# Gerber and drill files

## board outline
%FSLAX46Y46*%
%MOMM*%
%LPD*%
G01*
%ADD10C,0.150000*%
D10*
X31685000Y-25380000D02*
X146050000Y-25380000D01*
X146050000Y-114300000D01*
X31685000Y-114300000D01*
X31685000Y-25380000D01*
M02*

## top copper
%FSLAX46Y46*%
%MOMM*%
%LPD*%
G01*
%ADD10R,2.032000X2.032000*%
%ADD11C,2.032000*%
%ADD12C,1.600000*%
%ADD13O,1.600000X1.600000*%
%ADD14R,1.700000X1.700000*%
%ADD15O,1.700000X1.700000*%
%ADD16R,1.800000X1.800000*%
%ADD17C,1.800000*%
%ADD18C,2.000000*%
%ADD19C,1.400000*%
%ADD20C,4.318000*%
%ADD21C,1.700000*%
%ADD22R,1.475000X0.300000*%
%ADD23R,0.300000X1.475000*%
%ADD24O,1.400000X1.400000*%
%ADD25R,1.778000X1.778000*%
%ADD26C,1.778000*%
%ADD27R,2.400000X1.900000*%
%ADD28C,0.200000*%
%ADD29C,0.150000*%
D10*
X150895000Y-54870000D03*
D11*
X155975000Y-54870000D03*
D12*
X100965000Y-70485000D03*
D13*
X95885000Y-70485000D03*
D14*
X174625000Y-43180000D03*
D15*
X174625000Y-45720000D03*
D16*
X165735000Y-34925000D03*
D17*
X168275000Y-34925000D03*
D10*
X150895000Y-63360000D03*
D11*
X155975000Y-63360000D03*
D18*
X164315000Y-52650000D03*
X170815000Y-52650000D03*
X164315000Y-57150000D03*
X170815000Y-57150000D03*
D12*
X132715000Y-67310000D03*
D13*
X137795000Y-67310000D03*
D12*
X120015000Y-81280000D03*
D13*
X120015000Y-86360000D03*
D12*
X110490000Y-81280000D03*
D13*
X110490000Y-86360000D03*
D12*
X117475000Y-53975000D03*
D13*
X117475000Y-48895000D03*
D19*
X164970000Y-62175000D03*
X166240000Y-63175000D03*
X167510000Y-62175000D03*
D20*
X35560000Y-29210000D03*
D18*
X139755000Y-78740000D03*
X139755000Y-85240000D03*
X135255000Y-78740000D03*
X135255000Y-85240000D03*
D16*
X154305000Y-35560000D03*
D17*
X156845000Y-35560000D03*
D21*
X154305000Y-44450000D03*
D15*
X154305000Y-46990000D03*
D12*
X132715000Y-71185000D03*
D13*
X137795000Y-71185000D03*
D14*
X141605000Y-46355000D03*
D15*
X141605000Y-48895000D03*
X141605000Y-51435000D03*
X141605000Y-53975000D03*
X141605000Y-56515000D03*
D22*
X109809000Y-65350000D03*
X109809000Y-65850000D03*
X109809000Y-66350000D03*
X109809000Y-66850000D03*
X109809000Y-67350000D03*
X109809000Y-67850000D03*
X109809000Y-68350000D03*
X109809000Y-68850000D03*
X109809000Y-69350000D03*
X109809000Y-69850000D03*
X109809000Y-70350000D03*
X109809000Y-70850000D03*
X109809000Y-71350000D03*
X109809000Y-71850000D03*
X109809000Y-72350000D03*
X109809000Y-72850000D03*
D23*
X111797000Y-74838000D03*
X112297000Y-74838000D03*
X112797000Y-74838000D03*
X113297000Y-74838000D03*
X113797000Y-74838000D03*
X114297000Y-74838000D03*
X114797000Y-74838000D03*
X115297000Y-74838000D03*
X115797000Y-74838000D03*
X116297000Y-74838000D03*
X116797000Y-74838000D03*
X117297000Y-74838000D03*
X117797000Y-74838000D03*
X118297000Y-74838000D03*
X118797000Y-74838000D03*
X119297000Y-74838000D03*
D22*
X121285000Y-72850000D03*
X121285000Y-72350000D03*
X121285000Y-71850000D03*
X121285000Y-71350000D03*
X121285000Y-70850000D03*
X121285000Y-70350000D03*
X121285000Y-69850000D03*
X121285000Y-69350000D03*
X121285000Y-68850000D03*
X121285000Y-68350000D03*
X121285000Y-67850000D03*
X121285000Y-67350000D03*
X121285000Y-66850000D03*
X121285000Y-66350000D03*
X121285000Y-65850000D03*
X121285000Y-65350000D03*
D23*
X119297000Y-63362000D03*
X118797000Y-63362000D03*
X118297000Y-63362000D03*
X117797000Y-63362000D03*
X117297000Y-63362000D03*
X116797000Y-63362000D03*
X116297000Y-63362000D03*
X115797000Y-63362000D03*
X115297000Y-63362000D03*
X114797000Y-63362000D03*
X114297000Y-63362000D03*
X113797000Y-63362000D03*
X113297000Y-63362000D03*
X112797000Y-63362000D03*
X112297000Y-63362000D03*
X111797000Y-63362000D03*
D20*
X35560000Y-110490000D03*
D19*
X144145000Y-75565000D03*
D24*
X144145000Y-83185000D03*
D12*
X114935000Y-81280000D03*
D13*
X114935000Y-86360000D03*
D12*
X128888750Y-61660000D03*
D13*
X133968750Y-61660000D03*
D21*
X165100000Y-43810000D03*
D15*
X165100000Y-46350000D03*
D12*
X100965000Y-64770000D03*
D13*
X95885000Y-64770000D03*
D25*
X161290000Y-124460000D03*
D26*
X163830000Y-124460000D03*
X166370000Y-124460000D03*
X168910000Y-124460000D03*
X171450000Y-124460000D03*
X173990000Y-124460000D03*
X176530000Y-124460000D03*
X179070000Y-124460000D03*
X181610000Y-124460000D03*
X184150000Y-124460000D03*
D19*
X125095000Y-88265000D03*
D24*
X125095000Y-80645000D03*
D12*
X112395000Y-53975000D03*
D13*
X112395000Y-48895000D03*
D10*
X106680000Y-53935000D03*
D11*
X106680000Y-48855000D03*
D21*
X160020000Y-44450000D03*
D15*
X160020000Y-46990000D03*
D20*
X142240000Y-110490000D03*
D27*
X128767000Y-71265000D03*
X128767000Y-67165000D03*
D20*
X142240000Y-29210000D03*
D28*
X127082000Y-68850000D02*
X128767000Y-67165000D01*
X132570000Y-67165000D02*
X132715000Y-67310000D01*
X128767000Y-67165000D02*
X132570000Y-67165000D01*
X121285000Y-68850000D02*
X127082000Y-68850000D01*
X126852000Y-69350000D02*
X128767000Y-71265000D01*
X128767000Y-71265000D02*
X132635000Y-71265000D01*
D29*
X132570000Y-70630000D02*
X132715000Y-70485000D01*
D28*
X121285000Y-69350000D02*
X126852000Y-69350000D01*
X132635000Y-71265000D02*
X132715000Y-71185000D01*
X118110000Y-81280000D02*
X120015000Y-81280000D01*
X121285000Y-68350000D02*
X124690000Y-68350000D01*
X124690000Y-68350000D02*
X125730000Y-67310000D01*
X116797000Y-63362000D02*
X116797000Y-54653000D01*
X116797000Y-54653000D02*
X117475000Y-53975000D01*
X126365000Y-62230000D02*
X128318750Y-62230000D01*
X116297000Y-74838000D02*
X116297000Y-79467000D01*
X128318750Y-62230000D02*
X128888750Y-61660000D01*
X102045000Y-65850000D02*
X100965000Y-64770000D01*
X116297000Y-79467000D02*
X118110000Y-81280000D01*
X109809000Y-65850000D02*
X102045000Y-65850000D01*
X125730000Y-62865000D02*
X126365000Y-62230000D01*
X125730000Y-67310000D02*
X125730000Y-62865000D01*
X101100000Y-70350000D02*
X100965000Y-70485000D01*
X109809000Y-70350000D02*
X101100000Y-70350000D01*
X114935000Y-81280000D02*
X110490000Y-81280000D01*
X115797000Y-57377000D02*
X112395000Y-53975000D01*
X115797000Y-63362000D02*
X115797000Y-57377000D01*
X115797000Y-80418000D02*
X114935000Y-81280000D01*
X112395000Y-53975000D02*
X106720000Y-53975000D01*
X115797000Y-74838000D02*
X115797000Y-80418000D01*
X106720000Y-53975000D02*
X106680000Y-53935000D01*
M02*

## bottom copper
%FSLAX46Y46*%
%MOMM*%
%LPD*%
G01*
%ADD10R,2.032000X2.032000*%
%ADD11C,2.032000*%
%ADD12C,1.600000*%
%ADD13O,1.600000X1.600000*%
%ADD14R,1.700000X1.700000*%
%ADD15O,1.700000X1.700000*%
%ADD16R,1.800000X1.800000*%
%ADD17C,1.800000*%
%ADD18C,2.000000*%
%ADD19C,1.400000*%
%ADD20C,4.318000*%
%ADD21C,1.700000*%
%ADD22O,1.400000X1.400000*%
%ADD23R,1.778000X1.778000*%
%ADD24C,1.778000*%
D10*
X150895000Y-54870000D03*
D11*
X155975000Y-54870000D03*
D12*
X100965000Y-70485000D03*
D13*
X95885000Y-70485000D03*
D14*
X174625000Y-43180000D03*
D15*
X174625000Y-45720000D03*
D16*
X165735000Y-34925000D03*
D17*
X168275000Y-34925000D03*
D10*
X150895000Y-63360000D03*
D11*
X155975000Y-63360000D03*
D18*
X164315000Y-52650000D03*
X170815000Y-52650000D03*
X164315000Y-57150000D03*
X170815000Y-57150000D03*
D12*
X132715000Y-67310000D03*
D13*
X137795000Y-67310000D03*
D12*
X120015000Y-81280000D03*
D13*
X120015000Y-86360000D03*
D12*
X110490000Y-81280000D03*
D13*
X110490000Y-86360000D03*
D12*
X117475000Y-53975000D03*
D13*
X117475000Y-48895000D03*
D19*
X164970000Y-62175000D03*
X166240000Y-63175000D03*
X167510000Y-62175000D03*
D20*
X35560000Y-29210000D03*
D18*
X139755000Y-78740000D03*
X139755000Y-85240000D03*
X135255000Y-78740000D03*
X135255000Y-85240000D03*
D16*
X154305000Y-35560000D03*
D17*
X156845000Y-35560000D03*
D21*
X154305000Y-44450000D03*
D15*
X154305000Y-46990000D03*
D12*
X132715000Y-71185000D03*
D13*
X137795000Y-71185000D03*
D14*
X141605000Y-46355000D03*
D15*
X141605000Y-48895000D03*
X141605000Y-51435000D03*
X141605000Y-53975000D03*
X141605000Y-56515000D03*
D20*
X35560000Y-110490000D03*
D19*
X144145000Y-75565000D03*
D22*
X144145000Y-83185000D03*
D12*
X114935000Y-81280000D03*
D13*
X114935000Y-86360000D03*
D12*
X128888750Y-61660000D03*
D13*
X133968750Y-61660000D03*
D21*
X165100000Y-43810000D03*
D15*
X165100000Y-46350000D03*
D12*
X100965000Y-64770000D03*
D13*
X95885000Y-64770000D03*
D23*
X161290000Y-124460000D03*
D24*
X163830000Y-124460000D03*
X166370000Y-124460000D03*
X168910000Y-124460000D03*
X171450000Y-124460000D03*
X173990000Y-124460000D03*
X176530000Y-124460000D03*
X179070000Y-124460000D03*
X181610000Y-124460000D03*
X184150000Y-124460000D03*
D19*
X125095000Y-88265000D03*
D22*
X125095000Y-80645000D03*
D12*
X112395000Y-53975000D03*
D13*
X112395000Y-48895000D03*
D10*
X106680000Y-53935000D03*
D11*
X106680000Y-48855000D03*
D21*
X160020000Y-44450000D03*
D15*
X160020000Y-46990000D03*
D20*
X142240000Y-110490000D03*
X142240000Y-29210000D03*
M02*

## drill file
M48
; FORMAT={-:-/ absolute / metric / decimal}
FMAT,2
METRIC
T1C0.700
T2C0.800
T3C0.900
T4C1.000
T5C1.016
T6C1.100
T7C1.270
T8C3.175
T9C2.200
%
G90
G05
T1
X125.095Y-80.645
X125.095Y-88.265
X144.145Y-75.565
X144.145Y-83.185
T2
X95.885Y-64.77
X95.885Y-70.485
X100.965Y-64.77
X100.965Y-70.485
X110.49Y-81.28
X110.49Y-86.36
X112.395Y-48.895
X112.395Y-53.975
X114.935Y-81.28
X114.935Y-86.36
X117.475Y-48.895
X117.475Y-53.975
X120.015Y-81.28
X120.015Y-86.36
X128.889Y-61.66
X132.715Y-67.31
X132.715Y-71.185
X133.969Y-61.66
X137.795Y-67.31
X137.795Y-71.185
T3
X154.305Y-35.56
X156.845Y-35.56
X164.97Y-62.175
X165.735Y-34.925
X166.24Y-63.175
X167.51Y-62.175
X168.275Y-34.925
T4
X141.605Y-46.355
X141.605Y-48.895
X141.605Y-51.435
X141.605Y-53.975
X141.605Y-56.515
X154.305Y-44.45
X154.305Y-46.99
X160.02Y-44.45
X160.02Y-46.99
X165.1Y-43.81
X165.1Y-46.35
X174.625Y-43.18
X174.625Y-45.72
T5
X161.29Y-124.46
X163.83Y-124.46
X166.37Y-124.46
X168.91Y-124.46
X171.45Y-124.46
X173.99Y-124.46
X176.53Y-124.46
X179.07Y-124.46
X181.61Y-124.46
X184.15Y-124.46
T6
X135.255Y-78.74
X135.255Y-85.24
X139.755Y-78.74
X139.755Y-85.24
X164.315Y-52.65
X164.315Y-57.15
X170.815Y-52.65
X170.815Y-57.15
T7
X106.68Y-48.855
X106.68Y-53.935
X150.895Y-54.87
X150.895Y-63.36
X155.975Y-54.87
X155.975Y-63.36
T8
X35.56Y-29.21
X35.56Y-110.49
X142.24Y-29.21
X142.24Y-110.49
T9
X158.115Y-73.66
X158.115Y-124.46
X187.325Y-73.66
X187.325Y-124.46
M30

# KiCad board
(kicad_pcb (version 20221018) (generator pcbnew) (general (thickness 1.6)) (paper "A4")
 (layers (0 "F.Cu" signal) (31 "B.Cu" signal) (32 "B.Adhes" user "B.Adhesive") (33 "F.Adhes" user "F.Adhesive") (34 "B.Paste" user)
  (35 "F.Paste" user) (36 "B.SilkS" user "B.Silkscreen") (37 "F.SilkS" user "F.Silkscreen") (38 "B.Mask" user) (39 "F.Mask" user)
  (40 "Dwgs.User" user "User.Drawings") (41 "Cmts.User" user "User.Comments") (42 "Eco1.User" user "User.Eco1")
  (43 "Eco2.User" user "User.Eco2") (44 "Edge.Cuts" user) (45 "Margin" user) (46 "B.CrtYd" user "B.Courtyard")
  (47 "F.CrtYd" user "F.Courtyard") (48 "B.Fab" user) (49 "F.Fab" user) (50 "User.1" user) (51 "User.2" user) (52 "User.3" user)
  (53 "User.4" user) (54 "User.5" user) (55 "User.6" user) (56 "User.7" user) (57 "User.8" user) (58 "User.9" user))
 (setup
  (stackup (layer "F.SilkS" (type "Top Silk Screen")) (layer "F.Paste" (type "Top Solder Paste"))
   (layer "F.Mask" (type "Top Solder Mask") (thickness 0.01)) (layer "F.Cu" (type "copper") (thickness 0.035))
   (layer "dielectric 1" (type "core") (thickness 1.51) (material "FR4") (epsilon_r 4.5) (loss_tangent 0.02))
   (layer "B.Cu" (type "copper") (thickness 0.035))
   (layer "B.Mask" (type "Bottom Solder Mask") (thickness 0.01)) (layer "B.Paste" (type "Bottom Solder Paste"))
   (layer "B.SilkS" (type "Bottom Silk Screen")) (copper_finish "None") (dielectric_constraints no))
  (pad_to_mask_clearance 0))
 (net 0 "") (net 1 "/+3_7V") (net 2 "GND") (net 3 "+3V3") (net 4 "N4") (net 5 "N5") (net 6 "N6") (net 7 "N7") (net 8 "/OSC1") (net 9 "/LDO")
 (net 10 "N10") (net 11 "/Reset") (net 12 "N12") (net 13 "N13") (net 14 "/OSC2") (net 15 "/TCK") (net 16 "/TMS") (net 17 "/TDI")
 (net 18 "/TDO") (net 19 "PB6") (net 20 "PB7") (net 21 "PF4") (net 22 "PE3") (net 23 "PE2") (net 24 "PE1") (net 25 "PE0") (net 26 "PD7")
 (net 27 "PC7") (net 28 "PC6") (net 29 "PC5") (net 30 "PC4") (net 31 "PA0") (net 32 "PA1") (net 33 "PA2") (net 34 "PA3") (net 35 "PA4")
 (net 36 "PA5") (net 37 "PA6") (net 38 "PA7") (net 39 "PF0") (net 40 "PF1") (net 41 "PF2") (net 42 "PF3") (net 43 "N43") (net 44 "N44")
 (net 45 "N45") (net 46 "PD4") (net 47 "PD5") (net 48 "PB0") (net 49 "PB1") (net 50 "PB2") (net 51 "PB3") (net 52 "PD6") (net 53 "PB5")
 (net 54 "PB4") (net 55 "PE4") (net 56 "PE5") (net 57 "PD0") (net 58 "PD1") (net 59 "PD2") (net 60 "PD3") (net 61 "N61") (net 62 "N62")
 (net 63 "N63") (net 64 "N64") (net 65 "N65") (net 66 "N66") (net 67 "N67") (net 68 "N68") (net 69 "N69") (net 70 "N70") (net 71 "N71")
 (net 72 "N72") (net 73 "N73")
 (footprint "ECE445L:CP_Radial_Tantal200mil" (layer "F.Cu") (at 150.895 54.87)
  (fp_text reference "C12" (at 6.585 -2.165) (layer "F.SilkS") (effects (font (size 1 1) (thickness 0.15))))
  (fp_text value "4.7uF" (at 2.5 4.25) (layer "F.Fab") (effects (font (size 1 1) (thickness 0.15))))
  (pad "1" thru_hole rect (at 0 0) (size 2.032 2.032) (drill 1.27) (layers "*.Cu" "*.Mask") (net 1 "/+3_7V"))
  (pad "2" thru_hole circle (at 5.08 0) (size 2.032 2.032) (drill 1.27) (layers "*.Cu" "*.Mask") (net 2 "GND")))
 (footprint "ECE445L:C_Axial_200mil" (layer "F.Cu") (at 100.965 70.485 180)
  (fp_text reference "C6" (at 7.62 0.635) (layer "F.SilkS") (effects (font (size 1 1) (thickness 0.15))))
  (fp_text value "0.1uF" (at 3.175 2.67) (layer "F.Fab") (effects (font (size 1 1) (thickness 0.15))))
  (pad "1" thru_hole circle (at 0 0 180) (size 1.6 1.6) (drill 0.8) (layers "*.Cu" "*.Mask") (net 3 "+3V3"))
  (pad "2" thru_hole oval (at 5.08 0 180) (size 1.6 1.6) (drill 0.8) (layers "*.Cu" "*.Mask") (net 2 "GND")))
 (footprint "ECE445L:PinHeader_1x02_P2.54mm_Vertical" (layer "F.Cu") (at 174.625 43.18)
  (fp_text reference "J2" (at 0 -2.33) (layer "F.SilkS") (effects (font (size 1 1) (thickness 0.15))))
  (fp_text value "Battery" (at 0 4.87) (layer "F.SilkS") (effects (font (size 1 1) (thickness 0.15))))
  (pad "1" thru_hole rect (at 0 0) (size 1.7 1.7) (drill 1) (layers "*.Cu" "*.Mask") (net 2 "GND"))
  (pad "2" thru_hole oval (at 0 2.54) (size 1.7 1.7) (drill 1) (layers "*.Cu" "*.Mask") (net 1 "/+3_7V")))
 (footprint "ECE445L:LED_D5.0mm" (layer "F.Cu") (at 165.735 34.925)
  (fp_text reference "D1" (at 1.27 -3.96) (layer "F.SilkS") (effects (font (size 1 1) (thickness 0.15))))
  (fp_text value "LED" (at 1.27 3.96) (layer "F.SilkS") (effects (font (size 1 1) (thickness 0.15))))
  (pad "1" thru_hole rect (at 0 0) (size 1.8 1.8) (drill 0.9) (layers "*.Cu" "*.Mask") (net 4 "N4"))
  (pad "2" thru_hole circle (at 2.54 0) (size 1.8 1.8) (drill 0.9) (layers "*.Cu" "*.Mask") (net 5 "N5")))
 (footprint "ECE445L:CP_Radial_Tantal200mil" (layer "F.Cu") (at 150.895 63.36)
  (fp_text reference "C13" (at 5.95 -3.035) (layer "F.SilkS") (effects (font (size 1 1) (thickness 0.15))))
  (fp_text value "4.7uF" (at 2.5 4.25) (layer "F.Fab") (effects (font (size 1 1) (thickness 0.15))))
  (pad "1" thru_hole rect (at 0 0) (size 2.032 2.032) (drill 1.27) (layers "*.Cu" "*.Mask") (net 3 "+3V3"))
  (pad "2" thru_hole circle (at 5.08 0) (size 2.032 2.032) (drill 1.27) (layers "*.Cu" "*.Mask") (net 2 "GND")))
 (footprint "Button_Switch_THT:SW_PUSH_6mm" (layer "F.Cu") (at 164.315 52.65)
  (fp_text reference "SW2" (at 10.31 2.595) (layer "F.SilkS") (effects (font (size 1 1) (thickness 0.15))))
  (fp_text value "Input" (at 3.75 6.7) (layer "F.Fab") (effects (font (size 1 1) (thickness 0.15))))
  (pad "1" thru_hole circle (at 0 0 90) (size 2 2) (drill 1.1) (layers "*.Cu" "*.Mask") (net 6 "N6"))
  (pad "1" thru_hole circle (at 6.5 0 90) (size 2 2) (drill 1.1) (layers "*.Cu" "*.Mask") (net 6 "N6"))
  (pad "2" thru_hole circle (at 0 4.5 90) (size 2 2) (drill 1.1) (layers "*.Cu" "*.Mask") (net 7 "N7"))
  (pad "2" thru_hole circle (at 6.5 4.5 90) (size 2 2) (drill 1.1) (layers "*.Cu" "*.Mask") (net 7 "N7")))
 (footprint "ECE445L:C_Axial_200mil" (layer "F.Cu") (at 132.715 67.31)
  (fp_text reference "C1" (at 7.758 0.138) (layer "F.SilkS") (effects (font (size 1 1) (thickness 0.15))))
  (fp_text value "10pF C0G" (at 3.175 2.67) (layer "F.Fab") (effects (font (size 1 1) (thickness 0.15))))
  (pad "1" thru_hole circle (at 0 0) (size 1.6 1.6) (drill 0.8) (layers "*.Cu" "*.Mask") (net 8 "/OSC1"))
  (pad "2" thru_hole oval (at 5.08 0) (size 1.6 1.6) (drill 0.8) (layers "*.Cu" "*.Mask") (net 2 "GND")))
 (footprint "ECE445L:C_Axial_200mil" (layer "F.Cu") (at 120.015 81.28 -90)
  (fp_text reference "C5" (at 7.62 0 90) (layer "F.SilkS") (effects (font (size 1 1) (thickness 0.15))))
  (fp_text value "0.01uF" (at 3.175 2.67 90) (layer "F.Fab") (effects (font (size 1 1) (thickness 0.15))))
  (pad "1" thru_hole circle (at 0 0 270) (size 1.6 1.6) (drill 0.8) (layers "*.Cu" "*.Mask") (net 3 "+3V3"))
  (pad "2" thru_hole oval (at 5.08 0 270) (size 1.6 1.6) (drill 0.8) (layers "*.Cu" "*.Mask") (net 2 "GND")))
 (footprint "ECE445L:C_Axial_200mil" (layer "F.Cu") (at 110.49 81.28 -90)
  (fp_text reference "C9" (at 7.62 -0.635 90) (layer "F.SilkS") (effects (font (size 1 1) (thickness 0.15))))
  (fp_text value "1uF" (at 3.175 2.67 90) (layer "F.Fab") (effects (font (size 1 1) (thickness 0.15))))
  (pad "1" thru_hole circle (at 0 0 270) (size 1.6 1.6) (drill 0.8) (layers "*.Cu" "*.Mask") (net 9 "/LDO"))
  (pad "2" thru_hole oval (at 5.08 0 270) (size 1.6 1.6) (drill 0.8) (layers "*.Cu" "*.Mask") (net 2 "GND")))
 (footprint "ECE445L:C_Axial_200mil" (layer "F.Cu") (at 117.475 53.975 90)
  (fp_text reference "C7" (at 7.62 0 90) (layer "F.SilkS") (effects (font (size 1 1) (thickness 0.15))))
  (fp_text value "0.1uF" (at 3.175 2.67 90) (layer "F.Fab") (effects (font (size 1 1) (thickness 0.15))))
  (pad "1" thru_hole circle (at 0 0 90) (size 1.6 1.6) (drill 0.8) (layers "*.Cu" "*.Mask") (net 3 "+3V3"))
  (pad "2" thru_hole oval (at 5.08 0 90) (size 1.6 1.6) (drill 0.8) (layers "*.Cu" "*.Mask") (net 2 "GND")))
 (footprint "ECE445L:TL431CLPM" (layer "F.Cu") (at 164.97 62.175)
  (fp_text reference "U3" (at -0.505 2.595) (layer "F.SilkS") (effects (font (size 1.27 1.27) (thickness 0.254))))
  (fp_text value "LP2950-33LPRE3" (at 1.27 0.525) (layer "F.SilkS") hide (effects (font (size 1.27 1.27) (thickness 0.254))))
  (pad "1" thru_hole circle (at 0 0) (size 1.4 1.4) (drill 0.9) (layers "*.Cu" "*.Mask") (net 3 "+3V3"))
  (pad "2" thru_hole circle (at 1.27 1) (size 1.4 1.4) (drill 0.9) (layers "*.Cu" "*.Mask") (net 2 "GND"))
  (pad "3" thru_hole circle (at 2.54 0) (size 1.4 1.4) (drill 0.9) (layers "*.Cu" "*.Mask") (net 1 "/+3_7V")))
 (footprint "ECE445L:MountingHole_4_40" (layer "F.Cu") (at 35.56 29.21)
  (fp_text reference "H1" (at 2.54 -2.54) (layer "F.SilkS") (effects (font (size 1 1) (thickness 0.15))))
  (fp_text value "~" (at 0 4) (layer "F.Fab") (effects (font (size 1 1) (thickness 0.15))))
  (pad "1" thru_hole circle (at 0 0) (size 4.318 4.318) (drill 3.175) (layers "*.Cu" "*.Mask") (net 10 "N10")))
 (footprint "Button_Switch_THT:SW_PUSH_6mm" (layer "F.Cu") (at 139.755 78.74 -90)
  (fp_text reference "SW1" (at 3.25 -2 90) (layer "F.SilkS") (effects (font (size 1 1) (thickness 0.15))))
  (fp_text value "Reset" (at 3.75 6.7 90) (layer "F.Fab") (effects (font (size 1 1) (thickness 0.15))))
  (pad "1" thru_hole circle (at 0 0) (size 2 2) (drill 1.1) (layers "*.Cu" "*.Mask") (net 2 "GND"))
  (pad "1" thru_hole circle (at 6.5 0) (size 2 2) (drill 1.1) (layers "*.Cu" "*.Mask") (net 2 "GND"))
  (pad "2" thru_hole circle (at 0 4.5) (size 2 2) (drill 1.1) (layers "*.Cu" "*.Mask") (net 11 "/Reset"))
  (pad "2" thru_hole circle (at 6.5 4.5) (size 2 2) (drill 1.1) (layers "*.Cu" "*.Mask") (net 11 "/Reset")))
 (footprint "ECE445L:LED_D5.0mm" (layer "F.Cu") (at 154.305 35.56)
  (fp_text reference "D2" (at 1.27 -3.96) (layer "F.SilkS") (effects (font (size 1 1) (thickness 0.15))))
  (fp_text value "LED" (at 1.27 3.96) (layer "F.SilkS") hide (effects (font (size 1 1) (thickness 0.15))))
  (pad "1" thru_hole rect (at 0 0) (size 1.8 1.8) (drill 0.9) (layers "*.Cu" "*.Mask") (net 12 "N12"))
  (pad "2" thru_hole circle (at 2.54 0) (size 1.8 1.8) (drill 0.9) (layers "*.Cu" "*.Mask") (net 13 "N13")))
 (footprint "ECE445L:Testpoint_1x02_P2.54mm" (layer "F.Cu") (at 154.305 44.45)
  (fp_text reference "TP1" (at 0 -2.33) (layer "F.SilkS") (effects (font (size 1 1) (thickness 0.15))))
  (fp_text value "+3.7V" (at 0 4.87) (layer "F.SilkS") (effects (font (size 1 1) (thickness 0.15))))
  (pad "1" thru_hole circle (at 0 0) (size 1.7 1.7) (drill 1) (layers "*.Cu" "*.Mask") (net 1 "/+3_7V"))
  (pad "2" thru_hole oval (at 0 2.54) (size 1.7 1.7) (drill 1) (layers "*.Cu" "*.Mask") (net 1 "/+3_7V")))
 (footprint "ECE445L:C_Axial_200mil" (layer "F.Cu") (at 132.715 71.185)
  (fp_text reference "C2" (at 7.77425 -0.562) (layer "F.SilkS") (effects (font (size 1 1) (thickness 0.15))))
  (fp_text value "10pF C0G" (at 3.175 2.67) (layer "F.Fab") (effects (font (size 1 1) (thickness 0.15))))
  (pad "1" thru_hole circle (at 0 0) (size 1.6 1.6) (drill 0.8) (layers "*.Cu" "*.Mask") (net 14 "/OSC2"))
  (pad "2" thru_hole oval (at 5.08 0) (size 1.6 1.6) (drill 0.8) (layers "*.Cu" "*.Mask") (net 2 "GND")))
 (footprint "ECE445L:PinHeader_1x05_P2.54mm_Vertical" (layer "F.Cu") (at 141.605 46.355)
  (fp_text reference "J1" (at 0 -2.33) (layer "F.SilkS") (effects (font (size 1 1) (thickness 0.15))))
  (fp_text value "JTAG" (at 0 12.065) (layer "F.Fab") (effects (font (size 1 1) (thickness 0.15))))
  (pad "1" thru_hole rect (at 0 0) (size 1.7 1.7) (drill 1) (layers "*.Cu" "*.Mask") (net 2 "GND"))
  (pad "2" thru_hole oval (at 0 2.54) (size 1.7 1.7) (drill 1) (layers "*.Cu" "*.Mask") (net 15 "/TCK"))
  (pad "3" thru_hole oval (at 0 5.08) (size 1.7 1.7) (drill 1) (layers "*.Cu" "*.Mask") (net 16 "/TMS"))
  (pad "4" thru_hole oval (at 0 7.62) (size 1.7 1.7) (drill 1) (layers "*.Cu" "*.Mask") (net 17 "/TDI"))
  (pad "5" thru_hole oval (at 0 10.16) (size 1.7 1.7) (drill 1) (layers "*.Cu" "*.Mask") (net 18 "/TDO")))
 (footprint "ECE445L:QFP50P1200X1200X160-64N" (layer "F.Cu") (at 115.547 69.1)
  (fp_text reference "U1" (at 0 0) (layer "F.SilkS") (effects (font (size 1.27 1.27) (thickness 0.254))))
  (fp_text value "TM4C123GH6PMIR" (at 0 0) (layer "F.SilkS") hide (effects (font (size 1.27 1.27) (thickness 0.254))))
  (pad "1" smd rect (at -5.738 -3.75 90) (size 0.3 1.475) (layers "F.Cu" "F.Paste" "F.Mask") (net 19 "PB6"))
  (pad "2" smd rect (at -5.738 -3.25 90) (size 0.3 1.475) (layers "F.Cu" "F.Paste" "F.Mask") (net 3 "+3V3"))
  (pad "3" smd rect (at -5.738 -2.75 90) (size 0.3 1.475) (layers "F.Cu" "F.Paste" "F.Mask") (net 2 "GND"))
  (pad "4" smd rect (at -5.738 -2.25 90) (size 0.3 1.475) (layers "F.Cu" "F.Paste" "F.Mask") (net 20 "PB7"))
  (pad "5" smd rect (at -5.738 -1.75 90) (size 0.3 1.475) (layers "F.Cu" "F.Paste" "F.Mask") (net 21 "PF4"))
  (pad "6" smd rect (at -5.738 -1.25 90) (size 0.3 1.475) (layers "F.Cu" "F.Paste" "F.Mask") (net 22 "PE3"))
  (pad "7" smd rect (at -5.738 -0.75 90) (size 0.3 1.475) (layers "F.Cu" "F.Paste" "F.Mask") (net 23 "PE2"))
  (pad "8" smd rect (at -5.738 -0.25 90) (size 0.3 1.475) (layers "F.Cu" "F.Paste" "F.Mask") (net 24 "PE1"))
  (pad "9" smd rect (at -5.738 0.25 90) (size 0.3 1.475) (layers "F.Cu" "F.Paste" "F.Mask") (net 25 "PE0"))
  (pad "10" smd rect (at -5.738 0.75 90) (size 0.3 1.475) (layers "F.Cu" "F.Paste" "F.Mask") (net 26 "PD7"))
  (pad "11" smd rect (at -5.738 1.25 90) (size 0.3 1.475) (layers "F.Cu" "F.Paste" "F.Mask") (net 3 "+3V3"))
  (pad "12" smd rect (at -5.738 1.75 90) (size 0.3 1.475) (layers "F.Cu" "F.Paste" "F.Mask") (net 2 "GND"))
  (pad "13" smd rect (at -5.738 2.25 90) (size 0.3 1.475) (layers "F.Cu" "F.Paste" "F.Mask") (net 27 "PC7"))
  (pad "14" smd rect (at -5.738 2.75 90) (size 0.3 1.475) (layers "F.Cu" "F.Paste" "F.Mask") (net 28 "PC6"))
  (pad "15" smd rect (at -5.738 3.25 90) (size 0.3 1.475) (layers "F.Cu" "F.Paste" "F.Mask") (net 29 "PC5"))
  (pad "16" smd rect (at -5.738 3.75 90) (size 0.3 1.475) (layers "F.Cu" "F.Paste" "F.Mask") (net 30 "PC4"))
  (pad "17" smd rect (at -3.75 5.738) (size 0.3 1.475) (layers "F.Cu" "F.Paste" "F.Mask") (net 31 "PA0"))
  (pad "18" smd rect (at -3.25 5.738) (size 0.3 1.475) (layers "F.Cu" "F.Paste" "F.Mask") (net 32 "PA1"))
  (pad "19" smd rect (at -2.75 5.738) (size 0.3 1.475) (layers "F.Cu" "F.Paste" "F.Mask") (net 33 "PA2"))
  (pad "20" smd rect (at -2.25 5.738) (size 0.3 1.475) (layers "F.Cu" "F.Paste" "F.Mask") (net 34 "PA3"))
  (pad "21" smd rect (at -1.75 5.738) (size 0.3 1.475) (layers "F.Cu" "F.Paste" "F.Mask") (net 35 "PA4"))
  (pad "22" smd rect (at -1.25 5.738) (size 0.3 1.475) (layers "F.Cu" "F.Paste" "F.Mask") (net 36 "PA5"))
  (pad "23" smd rect (at -0.75 5.738) (size 0.3 1.475) (layers "F.Cu" "F.Paste" "F.Mask") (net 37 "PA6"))
  (pad "24" smd rect (at -0.25 5.738) (size 0.3 1.475) (layers "F.Cu" "F.Paste" "F.Mask") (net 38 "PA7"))
  (pad "25" smd rect (at 0.25 5.738) (size 0.3 1.475) (layers "F.Cu" "F.Paste" "F.Mask") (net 9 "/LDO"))
  (pad "26" smd rect (at 0.75 5.738) (size 0.3 1.475) (layers "F.Cu" "F.Paste" "F.Mask") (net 3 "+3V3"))
  (pad "27" smd rect (at 1.25 5.738) (size 0.3 1.475) (layers "F.Cu" "F.Paste" "F.Mask") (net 2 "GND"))
  (pad "28" smd rect (at 1.75 5.738) (size 0.3 1.475) (layers "F.Cu" "F.Paste" "F.Mask") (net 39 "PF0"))
  (pad "29" smd rect (at 2.25 5.738) (size 0.3 1.475) (layers "F.Cu" "F.Paste" "F.Mask") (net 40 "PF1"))
  (pad "30" smd rect (at 2.75 5.738) (size 0.3 1.475) (layers "F.Cu" "F.Paste" "F.Mask") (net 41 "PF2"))
  (pad "31" smd rect (at 3.25 5.738) (size 0.3 1.475) (layers "F.Cu" "F.Paste" "F.Mask") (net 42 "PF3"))
  (pad "32" smd rect (at 3.75 5.738) (size 0.3 1.475) (layers "F.Cu" "F.Paste" "F.Mask") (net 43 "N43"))
  (pad "33" smd rect (at 5.738 3.75 90) (size 0.3 1.475) (layers "F.Cu" "F.Paste" "F.Mask") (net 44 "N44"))
  (pad "34" smd rect (at 5.738 3.25 90) (size 0.3 1.475) (layers "F.Cu" "F.Paste" "F.Mask") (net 2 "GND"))
  (pad "35" smd rect (at 5.738 2.75 90) (size 0.3 1.475) (layers "F.Cu" "F.Paste" "F.Mask") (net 2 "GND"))
  (pad "36" smd rect (at 5.738 2.25 90) (size 0.3 1.475) (layers "F.Cu" "F.Paste" "F.Mask") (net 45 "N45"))
  (pad "37" smd rect (at 5.738 1.75 90) (size 0.3 1.475) (layers "F.Cu" "F.Paste" "F.Mask") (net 3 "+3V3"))
  (pad "38" smd rect (at 5.738 1.25 90) (size 0.3 1.475) (layers "F.Cu" "F.Paste" "F.Mask") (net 11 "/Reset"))
  (pad "39" smd rect (at 5.738 0.75 90) (size 0.3 1.475) (layers "F.Cu" "F.Paste" "F.Mask") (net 2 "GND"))
  (pad "40" smd rect (at 5.738 0.25 90) (size 0.3 1.475) (layers "F.Cu" "F.Paste" "F.Mask") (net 14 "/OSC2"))
  (pad "41" smd rect (at 5.738 -0.25 90) (size 0.3 1.475) (layers "F.Cu" "F.Paste" "F.Mask") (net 8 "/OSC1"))
  (pad "42" smd rect (at 5.738 -0.75 90) (size 0.3 1.475) (layers "F.Cu" "F.Paste" "F.Mask") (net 3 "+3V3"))
  (pad "43" smd rect (at 5.738 -1.25 90) (size 0.3 1.475) (layers "F.Cu" "F.Paste" "F.Mask") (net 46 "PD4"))
  (pad "44" smd rect (at 5.738 -1.75 90) (size 0.3 1.475) (layers "F.Cu" "F.Paste" "F.Mask") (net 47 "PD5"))
  (pad "45" smd rect (at 5.738 -2.25 90) (size 0.3 1.475) (layers "F.Cu" "F.Paste" "F.Mask") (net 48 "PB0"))
  (pad "46" smd rect (at 5.738 -2.75 90) (size 0.3 1.475) (layers "F.Cu" "F.Paste" "F.Mask") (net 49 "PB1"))
  (pad "47" smd rect (at 5.738 -3.25 90) (size 0.3 1.475) (layers "F.Cu" "F.Paste" "F.Mask") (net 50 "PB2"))
  (pad "48" smd rect (at 5.738 -3.75 90) (size 0.3 1.475) (layers "F.Cu" "F.Paste" "F.Mask") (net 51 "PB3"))
  (pad "49" smd rect (at 3.75 -5.738) (size 0.3 1.475) (layers "F.Cu" "F.Paste" "F.Mask") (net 18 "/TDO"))
  (pad "50" smd rect (at 3.25 -5.738) (size 0.3 1.475) (layers "F.Cu" "F.Paste" "F.Mask") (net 17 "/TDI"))
  (pad "51" smd rect (at 2.75 -5.738) (size 0.3 1.475) (layers "F.Cu" "F.Paste" "F.Mask") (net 16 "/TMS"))
  (pad "52" smd rect (at 2.25 -5.738) (size 0.3 1.475) (layers "F.Cu" "F.Paste" "F.Mask") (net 15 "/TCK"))
  (pad "53" smd rect (at 1.75 -5.738) (size 0.3 1.475) (layers "F.Cu" "F.Paste" "F.Mask") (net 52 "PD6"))
  (pad "54" smd rect (at 1.25 -5.738) (size 0.3 1.475) (layers "F.Cu" "F.Paste" "F.Mask") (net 3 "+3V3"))
  (pad "55" smd rect (at 0.75 -5.738) (size 0.3 1.475) (layers "F.Cu" "F.Paste" "F.Mask") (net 2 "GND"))
  (pad "56" smd rect (at 0.25 -5.738) (size 0.3 1.475) (layers "F.Cu" "F.Paste" "F.Mask") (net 9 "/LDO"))
  (pad "57" smd rect (at -0.25 -5.738) (size 0.3 1.475) (layers "F.Cu" "F.Paste" "F.Mask") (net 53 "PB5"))
  (pad "58" smd rect (at -0.75 -5.738) (size 0.3 1.475) (layers "F.Cu" "F.Paste" "F.Mask") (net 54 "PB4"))
  (pad "59" smd rect (at -1.25 -5.738) (size 0.3 1.475) (layers "F.Cu" "F.Paste" "F.Mask") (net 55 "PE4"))
  (pad "60" smd rect (at -1.75 -5.738) (size 0.3 1.475) (layers "F.Cu" "F.Paste" "F.Mask") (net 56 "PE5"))
  (pad "61" smd rect (at -2.25 -5.738) (size 0.3 1.475) (layers "F.Cu" "F.Paste" "F.Mask") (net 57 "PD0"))
  (pad "62" smd rect (at -2.75 -5.738) (size 0.3 1.475) (layers "F.Cu" "F.Paste" "F.Mask") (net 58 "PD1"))
  (pad "63" smd rect (at -3.25 -5.738) (size 0.3 1.475) (layers "F.Cu" "F.Paste" "F.Mask") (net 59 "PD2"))
  (pad "64" smd rect (at -3.75 -5.738) (size 0.3 1.475) (layers "F.Cu" "F.Paste" "F.Mask") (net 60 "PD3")))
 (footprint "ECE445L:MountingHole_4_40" (layer "F.Cu") (at 35.56 110.49)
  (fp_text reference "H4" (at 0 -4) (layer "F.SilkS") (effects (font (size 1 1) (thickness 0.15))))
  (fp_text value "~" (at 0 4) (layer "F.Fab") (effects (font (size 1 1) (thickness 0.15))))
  (pad "1" thru_hole circle (at 0 0) (size 4.318 4.318) (drill 3.175) (layers "*.Cu" "*.Mask") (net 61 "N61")))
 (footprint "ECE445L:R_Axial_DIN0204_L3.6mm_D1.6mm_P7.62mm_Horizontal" (layer "F.Cu") (at 144.145 75.565 -90)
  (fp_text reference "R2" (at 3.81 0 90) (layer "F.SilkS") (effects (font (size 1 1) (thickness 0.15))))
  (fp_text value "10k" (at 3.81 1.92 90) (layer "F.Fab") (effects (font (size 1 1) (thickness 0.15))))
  (pad "1" thru_hole circle (at 0 0 270) (size 1.4 1.4) (drill 0.7) (layers "*.Cu" "*.Mask") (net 3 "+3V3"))
  (pad "2" thru_hole oval (at 7.62 0 270) (size 1.4 1.4) (drill 0.7) (layers "*.Cu" "*.Mask") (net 11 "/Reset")))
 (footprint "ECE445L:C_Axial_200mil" (layer "F.Cu") (at 114.935 81.28 -90)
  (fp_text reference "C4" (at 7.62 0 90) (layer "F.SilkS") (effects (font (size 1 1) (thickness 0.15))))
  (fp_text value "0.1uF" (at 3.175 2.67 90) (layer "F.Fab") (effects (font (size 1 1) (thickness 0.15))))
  (pad "1" thru_hole circle (at 0 0 270) (size 1.6 1.6) (drill 0.8) (layers "*.Cu" "*.Mask") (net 9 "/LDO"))
  (pad "2" thru_hole oval (at 5.08 0 270) (size 1.6 1.6) (drill 0.8) (layers "*.Cu" "*.Mask") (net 2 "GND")))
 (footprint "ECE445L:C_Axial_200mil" (layer "F.Cu") (at 128.88875 61.66)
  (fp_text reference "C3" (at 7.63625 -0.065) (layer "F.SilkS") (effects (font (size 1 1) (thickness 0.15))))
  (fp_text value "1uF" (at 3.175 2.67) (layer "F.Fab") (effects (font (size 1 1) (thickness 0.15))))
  (pad "1" thru_hole circle (at 0 0) (size 1.6 1.6) (drill 0.8) (layers "*.Cu" "*.Mask") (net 3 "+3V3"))
  (pad "2" thru_hole oval (at 5.08 0) (size 1.6 1.6) (drill 0.8) (layers "*.Cu" "*.Mask") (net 2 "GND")))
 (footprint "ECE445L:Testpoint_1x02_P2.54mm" (layer "F.Cu") (at 165.1 43.81)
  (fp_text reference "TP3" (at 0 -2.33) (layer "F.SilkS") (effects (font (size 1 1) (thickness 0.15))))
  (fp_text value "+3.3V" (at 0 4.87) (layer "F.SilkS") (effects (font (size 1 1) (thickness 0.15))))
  (pad "1" thru_hole circle (at 0 0) (size 1.7 1.7) (drill 1) (layers "*.Cu" "*.Mask") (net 3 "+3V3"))
  (pad "2" thru_hole oval (at 0 2.54) (size 1.7 1.7) (drill 1) (layers "*.Cu" "*.Mask") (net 3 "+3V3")))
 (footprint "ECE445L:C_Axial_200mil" (layer "F.Cu") (at 100.965 64.77 180)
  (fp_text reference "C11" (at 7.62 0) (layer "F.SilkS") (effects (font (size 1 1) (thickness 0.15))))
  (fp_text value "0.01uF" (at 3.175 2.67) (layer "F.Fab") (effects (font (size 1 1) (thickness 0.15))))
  (pad "1" thru_hole circle (at 0 0 180) (size 1.6 1.6) (drill 0.8) (layers "*.Cu" "*.Mask") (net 3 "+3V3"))
  (pad "2" thru_hole oval (at 5.08 0 180) (size 1.6 1.6) (drill 0.8) (layers "*.Cu" "*.Mask") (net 2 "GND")))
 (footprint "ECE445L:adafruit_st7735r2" (layer "F.Cu") (at 172.72 99.06)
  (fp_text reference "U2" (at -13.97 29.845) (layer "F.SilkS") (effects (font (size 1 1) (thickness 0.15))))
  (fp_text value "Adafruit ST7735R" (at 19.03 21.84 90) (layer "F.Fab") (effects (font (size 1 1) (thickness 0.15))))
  (pad "" np_thru_hole circle (at -14.605 -25.4 90) (size 2.2 2.2) (drill 2.2) (layers "*.Cu" "*.Mask"))
  (pad "" np_thru_hole circle (at -14.605 25.4 90) (size 2.2 2.2) (drill 2.2) (layers "F&B.Cu" "*.Mask"))
  (pad "" np_thru_hole circle (at 14.605 -25.4 90) (size 2.2 2.2) (drill 2.2) (layers "F&B.Cu" "*.Mask"))
  (pad "" np_thru_hole circle (at 14.605 25.4 90) (size 2.2 2.2) (drill 2.2) (layers "F&B.Cu" "*.Mask"))
  (pad "1" thru_hole rect (at -11.43 25.4 90) (size 1.778 1.778) (drill 1.016) (layers "*.Cu" "*.Mask") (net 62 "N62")
   (solder_mask_margin 0.102))
  (pad "2" thru_hole circle (at -8.89 25.4 90) (size 1.778 1.778) (drill 1.016) (layers "*.Cu" "*.Mask") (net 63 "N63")
   (solder_mask_margin 0.102))
  (pad "3" thru_hole circle (at -6.35 25.4 90) (size 1.778 1.778) (drill 1.016) (layers "*.Cu" "*.Mask") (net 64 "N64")
   (solder_mask_margin 0.102))
  (pad "4" thru_hole circle (at -3.81 25.4 90) (size 1.778 1.778) (drill 1.016) (layers "*.Cu" "*.Mask") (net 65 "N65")
   (solder_mask_margin 0.102))
  (pad "5" thru_hole circle (at -1.27 25.4 90) (size 1.778 1.778) (drill 1.016) (layers "*.Cu" "*.Mask") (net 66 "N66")
   (solder_mask_margin 0.102))
  (pad "6" thru_hole circle (at 1.27 25.4 90) (size 1.778 1.778) (drill 1.016) (layers "*.Cu" "*.Mask") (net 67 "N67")
   (solder_mask_margin 0.102))
  (pad "7" thru_hole circle (at 3.81 25.4 90) (size 1.778 1.778) (drill 1.016) (layers "*.Cu" "*.Mask") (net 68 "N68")
   (solder_mask_margin 0.102))
  (pad "8" thru_hole circle (at 6.35 25.4 90) (size 1.778 1.778) (drill 1.016) (layers "*.Cu" "*.Mask") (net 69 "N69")
   (solder_mask_margin 0.102))
  (pad "9" thru_hole circle (at 8.89 25.4 90) (size 1.778 1.778) (drill 1.016) (layers "*.Cu" "*.Mask") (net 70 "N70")
   (solder_mask_margin 0.102))
  (pad "10" thru_hole circle (at 11.43 25.4 90) (size 1.778 1.778) (drill 1.016) (layers "*.Cu" "*.Mask") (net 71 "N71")
   (solder_mask_margin 0.102)))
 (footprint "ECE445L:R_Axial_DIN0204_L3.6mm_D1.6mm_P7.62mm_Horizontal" (layer "F.Cu") (at 125.095 88.265 90)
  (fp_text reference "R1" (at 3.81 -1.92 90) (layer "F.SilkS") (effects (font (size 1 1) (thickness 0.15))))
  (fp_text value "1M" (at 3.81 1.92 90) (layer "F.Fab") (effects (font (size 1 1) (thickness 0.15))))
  (pad "1" thru_hole circle (at 0 0 90) (size 1.4 1.4) (drill 0.7) (layers "*.Cu" "*.Mask") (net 3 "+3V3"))
  (pad "2" thru_hole oval (at 7.62 0 90) (size 1.4 1.4) (drill 0.7) (layers "*.Cu" "*.Mask") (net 43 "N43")))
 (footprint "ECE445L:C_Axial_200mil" (layer "F.Cu") (at 112.395 53.975 90)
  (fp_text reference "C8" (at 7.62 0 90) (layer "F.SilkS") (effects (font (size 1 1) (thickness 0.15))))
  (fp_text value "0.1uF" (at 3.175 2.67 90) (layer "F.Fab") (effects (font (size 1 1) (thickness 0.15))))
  (pad "1" thru_hole circle (at 0 0 90) (size 1.6 1.6) (drill 0.8) (layers "*.Cu" "*.Mask") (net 9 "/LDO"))
  (pad "2" thru_hole oval (at 5.08 0 90) (size 1.6 1.6) (drill 0.8) (layers "*.Cu" "*.Mask") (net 2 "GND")))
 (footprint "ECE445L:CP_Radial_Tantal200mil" (layer "F.Cu") (at 106.68 53.935 90)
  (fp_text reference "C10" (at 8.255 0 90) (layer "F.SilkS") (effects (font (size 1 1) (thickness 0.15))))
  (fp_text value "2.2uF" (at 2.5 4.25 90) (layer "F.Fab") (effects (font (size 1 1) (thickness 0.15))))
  (pad "1" thru_hole rect (at 0 0 90) (size 2.032 2.032) (drill 1.27) (layers "*.Cu" "*.Mask") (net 9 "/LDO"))
  (pad "2" thru_hole circle (at 5.08 0 90) (size 2.032 2.032) (drill 1.27) (layers "*.Cu" "*.Mask") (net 2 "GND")))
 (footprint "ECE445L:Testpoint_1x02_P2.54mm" (layer "F.Cu") (at 160.02 44.45)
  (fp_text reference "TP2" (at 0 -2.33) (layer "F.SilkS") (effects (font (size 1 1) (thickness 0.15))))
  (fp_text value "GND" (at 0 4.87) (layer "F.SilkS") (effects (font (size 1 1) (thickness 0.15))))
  (pad "1" thru_hole circle (at 0 0) (size 1.7 1.7) (drill 1) (layers "*.Cu" "*.Mask") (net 2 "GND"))
  (pad "2" thru_hole oval (at 0 2.54) (size 1.7 1.7) (drill 1) (layers "*.Cu" "*.Mask") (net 2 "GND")))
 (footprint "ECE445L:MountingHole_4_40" (layer "F.Cu") (at 142.24 110.49)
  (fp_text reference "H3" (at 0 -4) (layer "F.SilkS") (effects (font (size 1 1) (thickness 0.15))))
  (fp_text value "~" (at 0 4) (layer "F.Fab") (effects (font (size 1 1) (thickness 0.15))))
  (pad "1" thru_hole circle (at 0 0) (size 4.318 4.318) (drill 3.175) (layers "*.Cu" "*.Mask") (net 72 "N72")))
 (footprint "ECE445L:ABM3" (layer "F.Cu") (at 128.767 69.215 90)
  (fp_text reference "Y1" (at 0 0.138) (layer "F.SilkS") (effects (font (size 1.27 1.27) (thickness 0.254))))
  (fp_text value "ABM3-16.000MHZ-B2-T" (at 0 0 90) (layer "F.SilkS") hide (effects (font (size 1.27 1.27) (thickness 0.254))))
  (pad "1" smd rect (at -2.05 0 90) (size 1.9 2.4) (layers "F.Cu" "F.Paste" "F.Mask") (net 14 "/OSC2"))
  (pad "2" smd rect (at 2.05 0 90) (size 1.9 2.4) (layers "F.Cu" "F.Paste" "F.Mask") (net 8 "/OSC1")))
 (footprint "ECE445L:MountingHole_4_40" (layer "F.Cu") (at 142.24 29.21)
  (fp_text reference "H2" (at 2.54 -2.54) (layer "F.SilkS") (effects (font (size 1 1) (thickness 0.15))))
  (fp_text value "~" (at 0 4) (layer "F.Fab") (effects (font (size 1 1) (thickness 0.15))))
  (pad "1" thru_hole circle (at 0 0) (size 4.318 4.318) (drill 3.175) (layers "*.Cu" "*.Mask") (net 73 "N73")))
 (gr_rect (start 31.685 25.38) (end 146.05 114.3) (stroke (width 0.15) (type default)) (fill none) (layer "Edge.Cuts"))
 (segment (start 127.082 68.85) (end 128.767 67.165) (width 0.2) (layer "F.Cu") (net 8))
 (segment (start 132.57 67.165) (end 132.715 67.31) (width 0.2) (layer "F.Cu") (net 8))
 (segment (start 128.767 67.165) (end 132.57 67.165) (width 0.2) (layer "F.Cu") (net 8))
 (segment (start 121.285 68.85) (end 127.082 68.85) (width 0.2) (layer "F.Cu") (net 8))
 (segment (start 126.852 69.35) (end 128.767 71.265) (width 0.2) (layer "F.Cu") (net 14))
 (segment (start 128.767 71.265) (end 132.635 71.265) (width 0.2) (layer "F.Cu") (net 14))
 (segment (start 132.57 70.63) (end 132.715 70.485) (width 0.15) (layer "F.Cu") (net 14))
 (segment (start 121.285 69.35) (end 126.852 69.35) (width 0.2) (layer "F.Cu") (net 14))
 (segment (start 132.635 71.265) (end 132.715 71.185) (width 0.2) (layer "F.Cu") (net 14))
 (segment (start 118.11 81.28) (end 120.015 81.28) (width 0.2) (layer "F.Cu") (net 3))
 (segment (start 121.285 68.35) (end 124.69 68.35) (width 0.2) (layer "F.Cu") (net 3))
 (segment (start 124.69 68.35) (end 125.73 67.31) (width 0.2) (layer "F.Cu") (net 3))
 (segment (start 116.797 63.362) (end 116.797 54.653) (width 0.2) (layer "F.Cu") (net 3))
 (segment (start 116.797 54.653) (end 117.475 53.975) (width 0.2) (layer "F.Cu") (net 3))
 (segment (start 126.365 62.23) (end 128.31875 62.23) (width 0.2) (layer "F.Cu") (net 3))
 (segment (start 116.297 74.838) (end 116.297 79.467) (width 0.2) (layer "F.Cu") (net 3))
 (segment (start 128.31875 62.23) (end 128.88875 61.66) (width 0.2) (layer "F.Cu") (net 3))
 (segment (start 102.045 65.85) (end 100.965 64.77) (width 0.2) (layer "F.Cu") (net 3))
 (segment (start 116.297 79.467) (end 118.11 81.28) (width 0.2) (layer "F.Cu") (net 3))
 (segment (start 109.809 65.85) (end 102.045 65.85) (width 0.2) (layer "F.Cu") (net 3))
 (segment (start 125.73 62.865) (end 126.365 62.23) (width 0.2) (layer "F.Cu") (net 3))
 (segment (start 125.73 67.31) (end 125.73 62.865) (width 0.2) (layer "F.Cu") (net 3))
 (segment (start 101.1 70.35) (end 100.965 70.485) (width 0.2) (layer "F.Cu") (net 3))
 (segment (start 109.809 70.35) (end 101.1 70.35) (width 0.2) (layer "F.Cu") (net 3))
 (segment (start 114.935 81.28) (end 110.49 81.28) (width 0.2) (layer "F.Cu") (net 9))
 (segment (start 115.797 57.377) (end 112.395 53.975) (width 0.2) (layer "F.Cu") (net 9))
 (segment (start 115.797 63.362) (end 115.797 57.377) (width 0.2) (layer "F.Cu") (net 9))
 (segment (start 115.797 80.418) (end 114.935 81.28) (width 0.2) (layer "F.Cu") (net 9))
 (segment (start 112.395 53.975) (end 106.72 53.975) (width 0.2) (layer "F.Cu") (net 9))
 (segment (start 115.797 74.838) (end 115.797 80.418) (width 0.2) (layer "F.Cu") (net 9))
 (segment (start 106.72 53.975) (end 106.68 53.935) (width 0.2) (layer "F.Cu") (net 9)))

